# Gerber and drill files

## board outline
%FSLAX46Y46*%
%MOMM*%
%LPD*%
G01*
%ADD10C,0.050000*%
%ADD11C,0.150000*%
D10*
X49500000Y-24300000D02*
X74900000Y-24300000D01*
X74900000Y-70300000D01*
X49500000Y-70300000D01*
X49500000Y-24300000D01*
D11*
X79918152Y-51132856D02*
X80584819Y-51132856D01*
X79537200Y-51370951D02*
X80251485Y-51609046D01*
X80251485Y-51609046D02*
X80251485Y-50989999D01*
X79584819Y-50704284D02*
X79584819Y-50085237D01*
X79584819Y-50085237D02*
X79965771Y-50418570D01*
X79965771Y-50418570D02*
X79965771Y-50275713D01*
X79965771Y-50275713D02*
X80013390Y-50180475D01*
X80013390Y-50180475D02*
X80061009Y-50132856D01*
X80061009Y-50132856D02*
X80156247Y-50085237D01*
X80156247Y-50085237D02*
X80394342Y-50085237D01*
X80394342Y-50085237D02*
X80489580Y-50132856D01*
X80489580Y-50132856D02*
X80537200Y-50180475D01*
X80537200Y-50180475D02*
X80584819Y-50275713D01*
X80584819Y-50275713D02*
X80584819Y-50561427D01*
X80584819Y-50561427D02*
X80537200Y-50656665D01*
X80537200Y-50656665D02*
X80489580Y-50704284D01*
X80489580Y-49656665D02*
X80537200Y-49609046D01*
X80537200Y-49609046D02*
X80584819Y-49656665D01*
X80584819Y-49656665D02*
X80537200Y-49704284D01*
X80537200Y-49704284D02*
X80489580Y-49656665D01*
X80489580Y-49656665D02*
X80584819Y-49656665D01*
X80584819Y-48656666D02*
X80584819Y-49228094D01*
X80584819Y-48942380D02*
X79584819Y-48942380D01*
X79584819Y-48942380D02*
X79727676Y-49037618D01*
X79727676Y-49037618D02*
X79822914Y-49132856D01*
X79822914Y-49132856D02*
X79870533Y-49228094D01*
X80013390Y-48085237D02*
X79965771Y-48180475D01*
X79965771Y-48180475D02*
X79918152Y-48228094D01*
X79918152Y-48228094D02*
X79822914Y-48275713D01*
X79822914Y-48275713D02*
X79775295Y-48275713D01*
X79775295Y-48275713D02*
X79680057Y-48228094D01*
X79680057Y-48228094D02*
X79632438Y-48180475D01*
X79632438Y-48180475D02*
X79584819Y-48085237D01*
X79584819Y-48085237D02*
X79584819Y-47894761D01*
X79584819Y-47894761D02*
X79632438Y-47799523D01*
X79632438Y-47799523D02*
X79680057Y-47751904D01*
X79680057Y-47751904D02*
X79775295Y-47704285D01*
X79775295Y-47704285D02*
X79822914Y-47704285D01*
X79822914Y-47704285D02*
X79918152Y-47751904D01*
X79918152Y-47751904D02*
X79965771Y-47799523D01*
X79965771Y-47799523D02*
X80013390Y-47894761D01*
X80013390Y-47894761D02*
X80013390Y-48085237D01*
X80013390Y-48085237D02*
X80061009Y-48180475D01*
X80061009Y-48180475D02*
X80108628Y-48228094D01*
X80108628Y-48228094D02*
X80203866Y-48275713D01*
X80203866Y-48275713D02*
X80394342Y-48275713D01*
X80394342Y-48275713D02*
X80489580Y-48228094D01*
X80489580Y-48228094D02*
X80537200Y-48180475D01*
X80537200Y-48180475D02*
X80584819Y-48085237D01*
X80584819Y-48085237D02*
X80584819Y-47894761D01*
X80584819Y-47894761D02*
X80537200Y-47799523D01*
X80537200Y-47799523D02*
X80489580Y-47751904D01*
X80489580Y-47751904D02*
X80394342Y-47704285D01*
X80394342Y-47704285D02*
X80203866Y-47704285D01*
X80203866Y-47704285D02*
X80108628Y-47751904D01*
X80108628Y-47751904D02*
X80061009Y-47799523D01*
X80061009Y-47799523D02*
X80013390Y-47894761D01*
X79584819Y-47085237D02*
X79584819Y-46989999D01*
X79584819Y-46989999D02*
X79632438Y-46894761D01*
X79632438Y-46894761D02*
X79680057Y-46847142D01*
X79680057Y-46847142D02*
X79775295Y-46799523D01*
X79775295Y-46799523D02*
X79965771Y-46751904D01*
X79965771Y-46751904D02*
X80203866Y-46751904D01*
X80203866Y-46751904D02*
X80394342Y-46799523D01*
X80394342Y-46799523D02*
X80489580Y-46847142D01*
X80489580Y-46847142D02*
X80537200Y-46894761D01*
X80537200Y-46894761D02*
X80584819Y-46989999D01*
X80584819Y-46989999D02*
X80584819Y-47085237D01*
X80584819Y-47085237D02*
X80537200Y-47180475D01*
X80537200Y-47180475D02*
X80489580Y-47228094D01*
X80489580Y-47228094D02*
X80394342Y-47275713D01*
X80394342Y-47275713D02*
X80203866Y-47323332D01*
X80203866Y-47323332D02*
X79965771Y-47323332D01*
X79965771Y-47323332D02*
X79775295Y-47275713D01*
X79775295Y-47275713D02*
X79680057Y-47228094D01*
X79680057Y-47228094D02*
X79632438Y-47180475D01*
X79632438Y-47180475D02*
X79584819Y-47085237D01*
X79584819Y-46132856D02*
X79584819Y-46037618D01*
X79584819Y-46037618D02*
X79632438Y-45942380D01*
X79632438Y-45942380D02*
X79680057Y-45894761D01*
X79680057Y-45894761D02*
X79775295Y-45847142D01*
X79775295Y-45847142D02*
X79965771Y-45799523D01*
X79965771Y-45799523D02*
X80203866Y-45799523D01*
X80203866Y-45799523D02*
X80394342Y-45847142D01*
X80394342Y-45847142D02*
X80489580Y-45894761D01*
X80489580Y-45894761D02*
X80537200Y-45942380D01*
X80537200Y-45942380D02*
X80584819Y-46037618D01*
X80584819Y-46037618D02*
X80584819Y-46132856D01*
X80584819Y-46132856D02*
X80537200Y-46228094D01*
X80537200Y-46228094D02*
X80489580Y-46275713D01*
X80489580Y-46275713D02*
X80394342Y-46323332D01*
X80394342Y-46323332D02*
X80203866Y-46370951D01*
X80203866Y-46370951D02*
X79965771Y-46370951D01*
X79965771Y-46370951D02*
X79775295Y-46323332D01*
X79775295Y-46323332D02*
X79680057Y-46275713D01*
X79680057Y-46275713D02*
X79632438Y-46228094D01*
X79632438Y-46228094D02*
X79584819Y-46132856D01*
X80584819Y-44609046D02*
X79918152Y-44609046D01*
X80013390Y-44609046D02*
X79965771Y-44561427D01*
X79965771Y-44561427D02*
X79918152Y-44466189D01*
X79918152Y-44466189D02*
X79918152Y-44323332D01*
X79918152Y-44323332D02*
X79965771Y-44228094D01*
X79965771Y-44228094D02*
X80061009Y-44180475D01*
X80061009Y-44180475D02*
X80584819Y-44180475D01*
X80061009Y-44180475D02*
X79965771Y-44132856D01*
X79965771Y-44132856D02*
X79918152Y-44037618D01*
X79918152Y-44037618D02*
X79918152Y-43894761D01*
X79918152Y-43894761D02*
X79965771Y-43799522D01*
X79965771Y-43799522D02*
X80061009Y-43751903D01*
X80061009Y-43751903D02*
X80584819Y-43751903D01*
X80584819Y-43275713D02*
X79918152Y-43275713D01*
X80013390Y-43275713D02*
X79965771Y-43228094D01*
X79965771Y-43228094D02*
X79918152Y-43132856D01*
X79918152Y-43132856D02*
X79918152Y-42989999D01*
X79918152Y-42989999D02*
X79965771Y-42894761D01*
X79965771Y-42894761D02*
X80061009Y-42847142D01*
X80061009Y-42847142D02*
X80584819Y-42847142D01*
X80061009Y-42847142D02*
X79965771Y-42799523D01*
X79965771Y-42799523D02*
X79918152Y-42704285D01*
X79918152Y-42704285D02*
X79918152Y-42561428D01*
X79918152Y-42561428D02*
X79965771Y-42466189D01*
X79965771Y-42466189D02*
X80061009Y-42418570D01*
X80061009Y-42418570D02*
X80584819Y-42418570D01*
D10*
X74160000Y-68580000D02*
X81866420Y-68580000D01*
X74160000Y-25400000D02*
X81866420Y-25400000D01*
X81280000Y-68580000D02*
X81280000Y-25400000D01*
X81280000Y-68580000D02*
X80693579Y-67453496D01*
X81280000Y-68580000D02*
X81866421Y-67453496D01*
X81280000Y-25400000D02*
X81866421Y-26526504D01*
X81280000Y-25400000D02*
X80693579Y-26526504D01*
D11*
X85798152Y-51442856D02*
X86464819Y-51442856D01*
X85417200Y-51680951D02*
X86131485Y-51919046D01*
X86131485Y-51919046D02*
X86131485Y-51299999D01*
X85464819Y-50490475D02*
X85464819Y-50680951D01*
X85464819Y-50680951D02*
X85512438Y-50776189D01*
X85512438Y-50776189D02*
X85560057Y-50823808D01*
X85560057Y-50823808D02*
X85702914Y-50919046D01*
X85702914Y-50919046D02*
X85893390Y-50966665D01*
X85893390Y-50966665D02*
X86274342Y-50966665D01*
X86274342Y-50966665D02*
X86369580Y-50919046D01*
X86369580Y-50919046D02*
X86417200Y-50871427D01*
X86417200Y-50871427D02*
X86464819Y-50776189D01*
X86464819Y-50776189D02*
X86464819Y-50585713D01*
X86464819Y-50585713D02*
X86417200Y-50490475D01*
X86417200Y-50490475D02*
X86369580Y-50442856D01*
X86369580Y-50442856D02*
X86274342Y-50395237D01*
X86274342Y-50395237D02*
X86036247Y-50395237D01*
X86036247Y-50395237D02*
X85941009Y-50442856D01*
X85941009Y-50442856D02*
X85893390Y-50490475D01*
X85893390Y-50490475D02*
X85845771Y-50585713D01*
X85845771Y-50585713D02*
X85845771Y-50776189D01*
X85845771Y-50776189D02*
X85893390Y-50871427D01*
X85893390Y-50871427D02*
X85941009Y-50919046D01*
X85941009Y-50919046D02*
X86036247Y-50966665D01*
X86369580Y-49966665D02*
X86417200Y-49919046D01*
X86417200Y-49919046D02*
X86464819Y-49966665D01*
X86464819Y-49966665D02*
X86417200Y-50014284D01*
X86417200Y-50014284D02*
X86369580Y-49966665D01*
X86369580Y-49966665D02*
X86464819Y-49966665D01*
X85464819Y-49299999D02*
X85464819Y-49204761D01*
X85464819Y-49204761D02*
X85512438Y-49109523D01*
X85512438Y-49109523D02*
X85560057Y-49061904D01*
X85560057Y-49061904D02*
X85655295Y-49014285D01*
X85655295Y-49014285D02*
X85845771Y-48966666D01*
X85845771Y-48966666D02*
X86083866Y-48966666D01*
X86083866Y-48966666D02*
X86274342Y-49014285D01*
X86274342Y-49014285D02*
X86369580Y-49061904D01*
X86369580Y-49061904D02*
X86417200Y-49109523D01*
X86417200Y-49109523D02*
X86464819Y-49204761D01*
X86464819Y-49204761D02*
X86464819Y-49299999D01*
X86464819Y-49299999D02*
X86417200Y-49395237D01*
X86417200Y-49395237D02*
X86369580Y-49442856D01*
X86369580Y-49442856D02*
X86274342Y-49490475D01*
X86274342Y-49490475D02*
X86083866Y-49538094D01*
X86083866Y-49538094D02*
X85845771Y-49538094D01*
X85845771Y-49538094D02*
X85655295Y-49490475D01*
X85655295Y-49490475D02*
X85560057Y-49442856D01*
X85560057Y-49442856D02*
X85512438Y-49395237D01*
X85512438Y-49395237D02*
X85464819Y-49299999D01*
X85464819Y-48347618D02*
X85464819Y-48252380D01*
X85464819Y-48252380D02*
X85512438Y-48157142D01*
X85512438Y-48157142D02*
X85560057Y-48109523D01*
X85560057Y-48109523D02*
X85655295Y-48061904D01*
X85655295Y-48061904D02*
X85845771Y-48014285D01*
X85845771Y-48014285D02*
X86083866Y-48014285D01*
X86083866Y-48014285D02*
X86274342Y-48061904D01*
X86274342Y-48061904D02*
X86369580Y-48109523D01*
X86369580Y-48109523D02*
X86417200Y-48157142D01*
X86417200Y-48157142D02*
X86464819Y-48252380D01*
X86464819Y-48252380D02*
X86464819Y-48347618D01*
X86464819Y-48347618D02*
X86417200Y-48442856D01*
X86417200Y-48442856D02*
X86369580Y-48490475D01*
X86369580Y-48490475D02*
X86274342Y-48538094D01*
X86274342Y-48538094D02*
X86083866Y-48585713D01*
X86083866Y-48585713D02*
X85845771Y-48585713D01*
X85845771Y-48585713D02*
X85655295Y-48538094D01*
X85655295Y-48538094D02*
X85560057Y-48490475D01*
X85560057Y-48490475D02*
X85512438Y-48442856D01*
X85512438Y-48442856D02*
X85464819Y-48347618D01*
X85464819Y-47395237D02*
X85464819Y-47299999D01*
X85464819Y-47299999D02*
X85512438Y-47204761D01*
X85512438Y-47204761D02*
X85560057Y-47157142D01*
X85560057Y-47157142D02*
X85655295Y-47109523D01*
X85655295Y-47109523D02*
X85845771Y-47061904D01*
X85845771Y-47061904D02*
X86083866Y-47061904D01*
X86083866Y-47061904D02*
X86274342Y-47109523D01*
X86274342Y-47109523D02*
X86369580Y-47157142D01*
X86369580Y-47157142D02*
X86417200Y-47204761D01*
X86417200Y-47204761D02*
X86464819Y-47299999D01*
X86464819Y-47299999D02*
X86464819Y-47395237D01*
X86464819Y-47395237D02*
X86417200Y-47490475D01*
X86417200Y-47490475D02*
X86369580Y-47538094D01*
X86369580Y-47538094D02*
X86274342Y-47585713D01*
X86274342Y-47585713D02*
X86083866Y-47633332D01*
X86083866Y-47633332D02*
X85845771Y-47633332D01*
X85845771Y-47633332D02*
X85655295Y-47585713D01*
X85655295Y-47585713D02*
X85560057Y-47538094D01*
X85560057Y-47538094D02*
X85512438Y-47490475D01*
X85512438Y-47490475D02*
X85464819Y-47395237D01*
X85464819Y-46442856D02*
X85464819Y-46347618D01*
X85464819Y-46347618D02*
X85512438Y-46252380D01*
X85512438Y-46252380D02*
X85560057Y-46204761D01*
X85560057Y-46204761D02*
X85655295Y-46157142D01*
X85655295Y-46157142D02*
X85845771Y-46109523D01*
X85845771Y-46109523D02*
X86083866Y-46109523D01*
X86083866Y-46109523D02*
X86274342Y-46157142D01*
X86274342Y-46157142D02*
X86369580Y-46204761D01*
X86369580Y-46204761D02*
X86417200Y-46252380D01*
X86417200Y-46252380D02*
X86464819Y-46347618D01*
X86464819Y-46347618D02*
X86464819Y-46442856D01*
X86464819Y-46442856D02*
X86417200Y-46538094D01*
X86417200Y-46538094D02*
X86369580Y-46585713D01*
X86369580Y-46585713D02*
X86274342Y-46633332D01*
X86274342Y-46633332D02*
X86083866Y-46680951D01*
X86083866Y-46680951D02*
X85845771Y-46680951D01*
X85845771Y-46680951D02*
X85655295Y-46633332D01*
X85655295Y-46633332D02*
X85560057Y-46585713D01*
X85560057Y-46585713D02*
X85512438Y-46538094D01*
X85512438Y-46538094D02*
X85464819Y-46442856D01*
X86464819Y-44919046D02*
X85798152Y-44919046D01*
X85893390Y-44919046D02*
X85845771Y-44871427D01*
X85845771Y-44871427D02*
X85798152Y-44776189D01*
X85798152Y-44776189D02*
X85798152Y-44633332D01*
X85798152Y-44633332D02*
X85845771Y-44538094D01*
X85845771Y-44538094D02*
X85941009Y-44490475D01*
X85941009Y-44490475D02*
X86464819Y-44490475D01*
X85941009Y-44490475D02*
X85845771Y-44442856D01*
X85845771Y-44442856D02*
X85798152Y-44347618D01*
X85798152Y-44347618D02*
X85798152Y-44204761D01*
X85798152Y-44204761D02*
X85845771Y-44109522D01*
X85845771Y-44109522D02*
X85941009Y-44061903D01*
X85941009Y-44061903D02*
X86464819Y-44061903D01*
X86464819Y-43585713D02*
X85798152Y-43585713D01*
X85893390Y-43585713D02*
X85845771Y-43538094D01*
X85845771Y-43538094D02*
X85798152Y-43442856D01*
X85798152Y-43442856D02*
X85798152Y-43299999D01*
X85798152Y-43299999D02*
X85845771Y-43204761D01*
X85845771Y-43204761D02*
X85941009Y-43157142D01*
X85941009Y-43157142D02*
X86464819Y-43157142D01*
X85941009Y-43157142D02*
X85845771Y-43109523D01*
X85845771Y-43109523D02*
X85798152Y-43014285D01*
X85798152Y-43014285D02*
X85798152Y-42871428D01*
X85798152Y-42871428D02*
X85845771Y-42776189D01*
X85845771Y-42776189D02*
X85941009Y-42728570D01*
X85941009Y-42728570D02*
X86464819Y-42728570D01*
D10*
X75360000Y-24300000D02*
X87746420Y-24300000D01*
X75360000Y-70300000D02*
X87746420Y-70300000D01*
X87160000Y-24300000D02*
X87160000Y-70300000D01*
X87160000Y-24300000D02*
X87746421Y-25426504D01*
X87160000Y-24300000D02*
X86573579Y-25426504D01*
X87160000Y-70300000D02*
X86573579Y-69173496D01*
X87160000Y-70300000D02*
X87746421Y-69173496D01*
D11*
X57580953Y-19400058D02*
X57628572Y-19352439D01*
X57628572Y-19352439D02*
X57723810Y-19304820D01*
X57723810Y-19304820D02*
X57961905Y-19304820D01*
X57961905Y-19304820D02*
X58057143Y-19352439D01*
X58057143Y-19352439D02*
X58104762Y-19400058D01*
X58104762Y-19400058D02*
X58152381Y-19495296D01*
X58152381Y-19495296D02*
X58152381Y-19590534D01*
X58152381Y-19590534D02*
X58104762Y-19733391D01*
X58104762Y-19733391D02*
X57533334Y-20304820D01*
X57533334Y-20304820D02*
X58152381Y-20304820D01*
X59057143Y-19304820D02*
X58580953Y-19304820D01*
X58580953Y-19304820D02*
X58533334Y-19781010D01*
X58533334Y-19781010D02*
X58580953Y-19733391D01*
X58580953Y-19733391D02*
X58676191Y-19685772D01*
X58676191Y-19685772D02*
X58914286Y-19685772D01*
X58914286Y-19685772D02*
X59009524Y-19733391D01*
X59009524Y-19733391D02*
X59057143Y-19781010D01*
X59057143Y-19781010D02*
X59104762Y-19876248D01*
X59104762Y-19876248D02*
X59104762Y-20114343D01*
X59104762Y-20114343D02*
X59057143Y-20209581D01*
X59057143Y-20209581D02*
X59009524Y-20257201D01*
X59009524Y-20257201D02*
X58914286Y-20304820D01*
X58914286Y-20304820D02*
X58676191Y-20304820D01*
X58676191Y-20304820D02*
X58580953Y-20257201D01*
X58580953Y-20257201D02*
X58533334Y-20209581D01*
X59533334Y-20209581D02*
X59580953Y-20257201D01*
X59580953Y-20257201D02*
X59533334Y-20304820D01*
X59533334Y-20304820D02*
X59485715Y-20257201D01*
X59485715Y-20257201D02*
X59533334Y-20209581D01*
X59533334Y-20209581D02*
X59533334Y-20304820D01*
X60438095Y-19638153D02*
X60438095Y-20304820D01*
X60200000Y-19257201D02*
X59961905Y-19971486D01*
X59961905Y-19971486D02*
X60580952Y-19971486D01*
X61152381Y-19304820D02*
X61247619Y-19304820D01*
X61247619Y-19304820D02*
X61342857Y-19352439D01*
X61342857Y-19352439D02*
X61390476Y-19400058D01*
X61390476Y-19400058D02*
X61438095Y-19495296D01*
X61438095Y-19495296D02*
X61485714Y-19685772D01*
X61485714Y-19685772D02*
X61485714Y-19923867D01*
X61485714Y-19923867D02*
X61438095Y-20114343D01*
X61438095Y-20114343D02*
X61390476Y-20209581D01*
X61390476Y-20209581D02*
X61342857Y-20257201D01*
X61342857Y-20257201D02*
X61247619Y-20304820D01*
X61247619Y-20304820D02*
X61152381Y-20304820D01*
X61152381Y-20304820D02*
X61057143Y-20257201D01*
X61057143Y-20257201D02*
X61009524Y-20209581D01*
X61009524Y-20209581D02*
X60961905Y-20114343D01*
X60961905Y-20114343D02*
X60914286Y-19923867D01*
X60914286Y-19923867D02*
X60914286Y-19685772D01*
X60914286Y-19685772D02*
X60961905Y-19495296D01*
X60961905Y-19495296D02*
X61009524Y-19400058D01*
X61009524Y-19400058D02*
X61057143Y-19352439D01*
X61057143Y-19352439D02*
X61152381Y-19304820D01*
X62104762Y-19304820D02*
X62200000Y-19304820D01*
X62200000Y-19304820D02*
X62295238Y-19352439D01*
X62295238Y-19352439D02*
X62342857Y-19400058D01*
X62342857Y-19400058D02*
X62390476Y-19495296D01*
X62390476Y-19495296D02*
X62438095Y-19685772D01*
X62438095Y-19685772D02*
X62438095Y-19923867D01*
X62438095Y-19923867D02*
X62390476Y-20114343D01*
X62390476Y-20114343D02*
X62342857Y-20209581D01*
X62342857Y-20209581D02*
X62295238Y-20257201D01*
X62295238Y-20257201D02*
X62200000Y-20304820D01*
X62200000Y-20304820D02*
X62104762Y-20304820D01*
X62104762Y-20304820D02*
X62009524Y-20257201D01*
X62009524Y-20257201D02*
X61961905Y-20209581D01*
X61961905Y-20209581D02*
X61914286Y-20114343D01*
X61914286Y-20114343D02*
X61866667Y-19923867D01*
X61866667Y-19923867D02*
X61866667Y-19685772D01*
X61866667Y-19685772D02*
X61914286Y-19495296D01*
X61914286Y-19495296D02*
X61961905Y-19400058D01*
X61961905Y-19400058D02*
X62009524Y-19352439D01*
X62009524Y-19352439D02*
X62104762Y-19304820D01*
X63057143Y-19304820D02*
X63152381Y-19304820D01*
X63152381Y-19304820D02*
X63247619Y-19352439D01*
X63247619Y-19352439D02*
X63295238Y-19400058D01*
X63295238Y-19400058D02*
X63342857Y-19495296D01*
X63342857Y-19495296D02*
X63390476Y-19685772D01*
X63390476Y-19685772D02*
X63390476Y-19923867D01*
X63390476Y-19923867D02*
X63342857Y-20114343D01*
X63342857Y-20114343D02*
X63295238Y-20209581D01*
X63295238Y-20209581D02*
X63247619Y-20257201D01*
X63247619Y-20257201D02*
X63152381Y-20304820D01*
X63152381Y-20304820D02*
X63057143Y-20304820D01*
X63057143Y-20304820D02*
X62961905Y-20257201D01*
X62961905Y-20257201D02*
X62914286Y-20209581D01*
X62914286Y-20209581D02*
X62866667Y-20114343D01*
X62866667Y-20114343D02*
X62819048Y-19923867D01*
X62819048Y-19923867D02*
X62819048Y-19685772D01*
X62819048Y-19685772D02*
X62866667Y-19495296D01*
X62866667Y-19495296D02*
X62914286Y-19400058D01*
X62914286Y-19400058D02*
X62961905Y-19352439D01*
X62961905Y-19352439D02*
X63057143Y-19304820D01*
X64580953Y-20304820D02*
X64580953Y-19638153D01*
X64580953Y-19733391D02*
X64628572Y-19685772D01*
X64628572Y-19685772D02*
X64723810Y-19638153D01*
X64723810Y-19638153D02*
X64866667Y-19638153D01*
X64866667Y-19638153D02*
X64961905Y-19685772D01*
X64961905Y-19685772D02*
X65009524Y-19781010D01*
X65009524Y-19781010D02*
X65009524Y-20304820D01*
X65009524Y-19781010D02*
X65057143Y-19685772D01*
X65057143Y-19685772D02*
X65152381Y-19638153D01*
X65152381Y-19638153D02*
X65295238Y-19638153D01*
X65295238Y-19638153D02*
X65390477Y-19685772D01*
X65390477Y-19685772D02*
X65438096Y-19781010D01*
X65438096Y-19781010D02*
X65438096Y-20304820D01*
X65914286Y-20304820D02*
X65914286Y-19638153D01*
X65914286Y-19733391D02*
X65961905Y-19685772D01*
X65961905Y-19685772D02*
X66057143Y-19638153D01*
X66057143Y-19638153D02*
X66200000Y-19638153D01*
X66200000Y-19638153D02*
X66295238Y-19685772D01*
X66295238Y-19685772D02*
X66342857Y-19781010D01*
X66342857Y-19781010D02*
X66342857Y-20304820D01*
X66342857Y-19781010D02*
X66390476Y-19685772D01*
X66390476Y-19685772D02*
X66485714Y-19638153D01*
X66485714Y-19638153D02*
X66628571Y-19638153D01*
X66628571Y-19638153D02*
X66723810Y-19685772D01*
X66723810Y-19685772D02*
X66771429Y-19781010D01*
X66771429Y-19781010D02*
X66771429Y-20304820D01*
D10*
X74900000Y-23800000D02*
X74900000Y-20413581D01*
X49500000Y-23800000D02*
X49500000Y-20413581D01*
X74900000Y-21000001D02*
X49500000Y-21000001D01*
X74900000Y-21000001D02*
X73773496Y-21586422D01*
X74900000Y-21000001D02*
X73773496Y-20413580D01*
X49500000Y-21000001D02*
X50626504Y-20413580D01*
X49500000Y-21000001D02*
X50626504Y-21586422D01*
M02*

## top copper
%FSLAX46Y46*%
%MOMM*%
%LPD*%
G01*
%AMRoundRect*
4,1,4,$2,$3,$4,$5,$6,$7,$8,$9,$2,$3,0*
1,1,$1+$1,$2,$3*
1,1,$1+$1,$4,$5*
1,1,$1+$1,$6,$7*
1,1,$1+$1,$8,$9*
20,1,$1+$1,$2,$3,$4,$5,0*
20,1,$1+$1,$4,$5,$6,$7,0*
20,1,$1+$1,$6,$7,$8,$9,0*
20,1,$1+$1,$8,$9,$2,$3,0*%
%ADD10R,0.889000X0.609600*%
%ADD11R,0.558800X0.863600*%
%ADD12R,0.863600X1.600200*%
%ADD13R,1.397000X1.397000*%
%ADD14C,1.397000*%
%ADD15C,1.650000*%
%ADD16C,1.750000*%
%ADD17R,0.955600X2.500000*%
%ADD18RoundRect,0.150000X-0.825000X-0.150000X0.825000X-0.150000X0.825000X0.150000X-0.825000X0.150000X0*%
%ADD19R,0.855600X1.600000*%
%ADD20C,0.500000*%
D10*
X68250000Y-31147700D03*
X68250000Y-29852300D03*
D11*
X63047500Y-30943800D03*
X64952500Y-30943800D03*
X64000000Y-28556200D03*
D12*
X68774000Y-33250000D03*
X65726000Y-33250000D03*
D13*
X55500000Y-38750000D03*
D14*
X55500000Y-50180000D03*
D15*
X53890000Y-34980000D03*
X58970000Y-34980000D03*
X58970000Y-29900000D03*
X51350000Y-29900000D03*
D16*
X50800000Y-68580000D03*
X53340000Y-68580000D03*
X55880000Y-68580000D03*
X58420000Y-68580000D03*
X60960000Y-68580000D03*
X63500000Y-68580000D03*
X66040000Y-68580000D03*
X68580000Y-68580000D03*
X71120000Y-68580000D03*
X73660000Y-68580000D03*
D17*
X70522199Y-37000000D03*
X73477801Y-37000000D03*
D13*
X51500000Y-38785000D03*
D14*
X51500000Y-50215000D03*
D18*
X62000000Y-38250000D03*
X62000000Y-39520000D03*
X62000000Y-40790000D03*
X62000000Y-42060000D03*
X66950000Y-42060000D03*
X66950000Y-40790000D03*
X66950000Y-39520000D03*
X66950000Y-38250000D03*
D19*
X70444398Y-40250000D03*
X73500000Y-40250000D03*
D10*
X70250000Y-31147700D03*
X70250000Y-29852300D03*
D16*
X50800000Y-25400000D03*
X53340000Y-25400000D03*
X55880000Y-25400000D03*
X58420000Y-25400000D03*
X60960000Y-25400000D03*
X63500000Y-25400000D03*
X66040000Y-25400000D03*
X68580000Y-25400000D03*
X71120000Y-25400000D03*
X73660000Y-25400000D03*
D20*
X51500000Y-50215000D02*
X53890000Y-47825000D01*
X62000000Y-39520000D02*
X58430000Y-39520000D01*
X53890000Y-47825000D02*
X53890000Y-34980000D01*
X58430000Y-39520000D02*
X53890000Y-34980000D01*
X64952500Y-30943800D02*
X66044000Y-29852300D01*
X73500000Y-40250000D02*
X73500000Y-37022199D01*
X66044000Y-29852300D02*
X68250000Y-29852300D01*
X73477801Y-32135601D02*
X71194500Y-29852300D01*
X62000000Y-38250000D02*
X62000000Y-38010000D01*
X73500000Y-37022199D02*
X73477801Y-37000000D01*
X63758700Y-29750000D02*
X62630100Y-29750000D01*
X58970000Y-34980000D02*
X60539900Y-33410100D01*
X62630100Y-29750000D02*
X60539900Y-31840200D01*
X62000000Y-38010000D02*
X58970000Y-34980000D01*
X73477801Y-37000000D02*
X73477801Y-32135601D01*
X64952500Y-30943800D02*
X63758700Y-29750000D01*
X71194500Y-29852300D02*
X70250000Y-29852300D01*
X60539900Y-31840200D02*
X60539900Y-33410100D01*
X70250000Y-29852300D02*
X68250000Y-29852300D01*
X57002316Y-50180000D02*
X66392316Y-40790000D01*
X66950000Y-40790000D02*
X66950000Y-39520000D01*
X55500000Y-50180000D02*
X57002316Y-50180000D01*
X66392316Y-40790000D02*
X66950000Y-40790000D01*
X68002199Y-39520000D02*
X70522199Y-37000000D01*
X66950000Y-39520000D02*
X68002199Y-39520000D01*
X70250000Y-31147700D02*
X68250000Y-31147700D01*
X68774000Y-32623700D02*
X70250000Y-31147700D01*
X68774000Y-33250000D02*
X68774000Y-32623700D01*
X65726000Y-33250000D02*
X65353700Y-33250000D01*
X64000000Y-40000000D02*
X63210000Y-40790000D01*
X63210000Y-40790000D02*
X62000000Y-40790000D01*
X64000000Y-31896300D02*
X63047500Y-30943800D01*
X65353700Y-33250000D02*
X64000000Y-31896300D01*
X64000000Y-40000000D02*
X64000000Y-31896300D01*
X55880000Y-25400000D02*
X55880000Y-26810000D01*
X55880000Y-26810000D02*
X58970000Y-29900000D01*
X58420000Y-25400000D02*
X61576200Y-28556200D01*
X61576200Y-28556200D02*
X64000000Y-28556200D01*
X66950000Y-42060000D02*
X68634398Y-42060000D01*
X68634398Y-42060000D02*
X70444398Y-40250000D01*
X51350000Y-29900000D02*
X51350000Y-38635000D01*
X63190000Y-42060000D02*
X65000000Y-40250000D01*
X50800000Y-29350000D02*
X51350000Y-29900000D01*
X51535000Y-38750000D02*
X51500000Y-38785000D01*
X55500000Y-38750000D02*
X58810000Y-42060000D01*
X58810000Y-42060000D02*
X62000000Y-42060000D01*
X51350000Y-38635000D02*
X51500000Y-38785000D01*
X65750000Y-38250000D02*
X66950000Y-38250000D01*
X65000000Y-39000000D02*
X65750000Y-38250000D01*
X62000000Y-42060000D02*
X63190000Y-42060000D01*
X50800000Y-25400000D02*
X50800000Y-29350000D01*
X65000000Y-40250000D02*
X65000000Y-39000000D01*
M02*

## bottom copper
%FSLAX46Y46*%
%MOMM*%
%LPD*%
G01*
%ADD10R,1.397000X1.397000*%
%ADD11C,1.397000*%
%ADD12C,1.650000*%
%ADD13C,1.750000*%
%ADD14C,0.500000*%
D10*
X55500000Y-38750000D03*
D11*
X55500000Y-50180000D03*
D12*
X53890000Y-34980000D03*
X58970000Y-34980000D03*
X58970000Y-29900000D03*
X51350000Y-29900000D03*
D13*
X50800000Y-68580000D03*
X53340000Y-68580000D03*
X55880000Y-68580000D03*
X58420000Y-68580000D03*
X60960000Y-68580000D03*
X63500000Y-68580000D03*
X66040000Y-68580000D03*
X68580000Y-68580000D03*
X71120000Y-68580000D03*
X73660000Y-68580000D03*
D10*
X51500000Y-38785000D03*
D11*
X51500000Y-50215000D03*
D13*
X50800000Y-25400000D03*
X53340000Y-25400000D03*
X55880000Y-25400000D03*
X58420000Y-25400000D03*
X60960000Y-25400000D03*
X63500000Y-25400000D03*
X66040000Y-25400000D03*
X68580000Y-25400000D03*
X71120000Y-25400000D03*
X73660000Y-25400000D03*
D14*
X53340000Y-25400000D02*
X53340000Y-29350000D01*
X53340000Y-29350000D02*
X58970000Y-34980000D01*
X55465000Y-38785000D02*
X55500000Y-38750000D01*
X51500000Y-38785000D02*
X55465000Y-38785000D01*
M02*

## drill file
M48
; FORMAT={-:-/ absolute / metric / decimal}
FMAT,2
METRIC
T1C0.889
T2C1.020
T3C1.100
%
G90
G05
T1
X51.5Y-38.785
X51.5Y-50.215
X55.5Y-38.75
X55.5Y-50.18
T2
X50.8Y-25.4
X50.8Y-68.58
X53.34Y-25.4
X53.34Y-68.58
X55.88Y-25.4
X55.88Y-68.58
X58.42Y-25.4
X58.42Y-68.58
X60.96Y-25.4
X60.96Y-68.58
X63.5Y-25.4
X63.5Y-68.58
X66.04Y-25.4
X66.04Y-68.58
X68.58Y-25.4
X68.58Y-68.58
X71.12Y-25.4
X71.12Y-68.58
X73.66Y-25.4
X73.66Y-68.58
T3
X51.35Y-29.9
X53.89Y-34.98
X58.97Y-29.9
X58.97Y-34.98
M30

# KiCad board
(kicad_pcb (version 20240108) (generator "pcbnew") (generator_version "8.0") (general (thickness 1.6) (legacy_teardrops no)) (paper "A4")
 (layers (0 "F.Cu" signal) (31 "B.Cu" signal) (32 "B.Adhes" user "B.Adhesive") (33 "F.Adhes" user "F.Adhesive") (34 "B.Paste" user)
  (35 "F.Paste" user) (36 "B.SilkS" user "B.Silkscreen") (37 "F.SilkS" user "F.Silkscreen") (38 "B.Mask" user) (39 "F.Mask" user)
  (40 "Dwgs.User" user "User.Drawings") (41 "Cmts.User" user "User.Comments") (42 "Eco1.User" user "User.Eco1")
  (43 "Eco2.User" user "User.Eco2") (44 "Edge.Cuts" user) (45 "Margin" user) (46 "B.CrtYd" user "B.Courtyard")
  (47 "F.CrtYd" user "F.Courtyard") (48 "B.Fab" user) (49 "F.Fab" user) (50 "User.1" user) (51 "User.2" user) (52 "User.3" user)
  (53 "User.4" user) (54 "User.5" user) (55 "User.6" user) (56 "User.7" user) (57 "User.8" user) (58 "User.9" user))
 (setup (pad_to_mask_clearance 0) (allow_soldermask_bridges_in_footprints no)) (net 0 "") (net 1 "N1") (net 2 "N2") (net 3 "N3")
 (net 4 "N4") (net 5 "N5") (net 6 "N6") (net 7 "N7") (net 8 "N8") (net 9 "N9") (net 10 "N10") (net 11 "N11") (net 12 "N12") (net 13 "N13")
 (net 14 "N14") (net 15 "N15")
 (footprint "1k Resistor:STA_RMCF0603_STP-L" (layer "F.Cu") (at 68.25 30.5 90)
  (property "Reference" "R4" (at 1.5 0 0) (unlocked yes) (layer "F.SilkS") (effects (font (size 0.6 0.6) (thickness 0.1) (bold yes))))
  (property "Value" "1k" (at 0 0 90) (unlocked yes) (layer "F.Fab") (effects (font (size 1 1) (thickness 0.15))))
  (pad "1" smd rect (at -0.6477 0 90) (size 0.6096 0.889) (layers "F.Cu" "F.Paste" "F.Mask") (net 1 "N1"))
  (pad "2" smd rect (at 0.6477 0 90) (size 0.6096 0.889) (layers "F.Cu" "F.Paste" "F.Mask") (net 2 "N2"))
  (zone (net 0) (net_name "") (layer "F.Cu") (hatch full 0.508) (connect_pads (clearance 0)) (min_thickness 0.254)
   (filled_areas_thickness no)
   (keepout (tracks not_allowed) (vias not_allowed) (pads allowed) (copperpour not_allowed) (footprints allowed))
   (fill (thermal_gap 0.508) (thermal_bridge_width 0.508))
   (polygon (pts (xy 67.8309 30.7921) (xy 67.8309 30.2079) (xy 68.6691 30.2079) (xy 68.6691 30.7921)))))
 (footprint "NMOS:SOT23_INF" (layer "F.Cu") (at 64 29.75)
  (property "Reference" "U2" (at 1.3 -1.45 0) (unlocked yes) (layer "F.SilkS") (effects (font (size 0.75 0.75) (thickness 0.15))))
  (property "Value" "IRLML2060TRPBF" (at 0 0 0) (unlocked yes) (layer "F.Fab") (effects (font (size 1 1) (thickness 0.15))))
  (pad "1" smd rect (at -0.9525 1.1938) (size 0.5588 0.8636) (layers "F.Cu" "F.Paste" "F.Mask") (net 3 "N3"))
  (pad "2" smd rect (at 0.9525 1.1938) (size 0.5588 0.8636) (layers "F.Cu" "F.Paste" "F.Mask") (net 2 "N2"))
  (pad "3" smd rect (at 0 -1.1938) (size 0.5588 0.8636) (layers "F.Cu" "F.Paste" "F.Mask") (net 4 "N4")))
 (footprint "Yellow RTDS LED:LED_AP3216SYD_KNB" (layer "F.Cu") (at 67.25 33.25 180)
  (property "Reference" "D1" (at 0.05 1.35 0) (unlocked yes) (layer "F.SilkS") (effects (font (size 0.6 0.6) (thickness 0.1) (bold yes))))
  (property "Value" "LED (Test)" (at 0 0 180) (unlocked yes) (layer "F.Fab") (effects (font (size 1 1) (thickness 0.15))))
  (pad "1" smd rect (at -1.524 0 180) (size 0.8636 1.6002) (layers "F.Cu" "F.Paste" "F.Mask") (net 1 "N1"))
  (pad "2" smd rect (at 1.524 0 180) (size 0.8636 1.6002) (layers "F.Cu" "F.Paste" "F.Mask") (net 3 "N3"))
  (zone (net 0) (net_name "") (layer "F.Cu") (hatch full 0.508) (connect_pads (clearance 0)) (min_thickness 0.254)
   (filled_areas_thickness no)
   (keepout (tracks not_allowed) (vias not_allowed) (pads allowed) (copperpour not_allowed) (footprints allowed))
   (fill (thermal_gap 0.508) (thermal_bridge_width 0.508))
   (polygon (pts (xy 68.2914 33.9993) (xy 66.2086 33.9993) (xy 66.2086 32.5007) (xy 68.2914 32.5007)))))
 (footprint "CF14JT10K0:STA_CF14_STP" (layer "F.Cu") (at 55.5 38.75 -90)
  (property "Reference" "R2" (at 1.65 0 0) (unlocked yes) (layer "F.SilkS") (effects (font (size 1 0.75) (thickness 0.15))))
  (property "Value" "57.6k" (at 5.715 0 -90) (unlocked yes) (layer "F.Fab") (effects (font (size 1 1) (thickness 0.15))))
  (pad "1" thru_hole rect (at 0 0 270) (size 1.397 1.397) (drill 0.889) (layers "*.Cu" "*.Mask") (remove_unused_layers no) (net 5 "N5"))
  (pad "2" thru_hole circle (at 11.43 0 270) (size 1.397 1.397) (drill 0.889) (layers "*.Cu" "*.Mask") (remove_unused_layers no)
   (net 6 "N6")))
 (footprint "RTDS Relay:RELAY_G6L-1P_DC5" (layer "F.Cu") (at 55.16 32.44)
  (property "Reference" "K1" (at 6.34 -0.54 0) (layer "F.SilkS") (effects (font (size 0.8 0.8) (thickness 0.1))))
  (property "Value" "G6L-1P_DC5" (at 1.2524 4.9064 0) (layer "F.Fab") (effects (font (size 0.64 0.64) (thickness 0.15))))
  (pad "2" thru_hole circle (at -1.27 2.54) (size 1.65 1.65) (drill 1.1) (layers "*.Cu" "*.Mask") (remove_unused_layers no) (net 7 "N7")
   (solder_mask_margin 0.102))
  (pad "4" thru_hole circle (at 3.81 2.54) (size 1.65 1.65) (drill 1.1) (layers "*.Cu" "*.Mask") (remove_unused_layers no) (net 2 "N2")
   (solder_mask_margin 0.102))
  (pad "5" thru_hole circle (at 3.81 -2.54) (size 1.65 1.65) (drill 1.1) (layers "*.Cu" "*.Mask") (remove_unused_layers no) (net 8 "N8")
   (solder_mask_margin 0.102))
  (pad "8" thru_hole circle (at -3.81 -2.54) (size 1.65 1.65) (drill 1.1) (layers "*.Cu" "*.Mask") (remove_unused_layers no) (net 5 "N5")
   (solder_mask_margin 0.102)))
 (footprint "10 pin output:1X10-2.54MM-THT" (layer "F.Cu") (at 50.8 68.58)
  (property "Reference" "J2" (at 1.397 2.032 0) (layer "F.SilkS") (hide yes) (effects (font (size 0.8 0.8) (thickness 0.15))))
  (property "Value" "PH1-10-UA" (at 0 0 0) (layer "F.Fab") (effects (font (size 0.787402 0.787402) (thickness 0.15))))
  (pad "1" thru_hole circle (at 0 0) (size 1.75 1.75) (drill 1.02) (layers "*.Cu" "*.Mask") (remove_unused_layers no)
   (solder_mask_margin 0.102))
  (pad "2" thru_hole circle (at 2.54 0) (size 1.75 1.75) (drill 1.02) (layers "*.Cu" "*.Mask") (remove_unused_layers no)
   (solder_mask_margin 0.102))
  (pad "3" thru_hole circle (at 5.08 0) (size 1.75 1.75) (drill 1.02) (layers "*.Cu" "*.Mask") (remove_unused_layers no)
   (solder_mask_margin 0.102))
  (pad "4" thru_hole circle (at 7.62 0) (size 1.75 1.75) (drill 1.02) (layers "*.Cu" "*.Mask") (remove_unused_layers no)
   (solder_mask_margin 0.102))
  (pad "5" thru_hole circle (at 10.16 0) (size 1.75 1.75) (drill 1.02) (layers "*.Cu" "*.Mask") (remove_unused_layers no)
   (solder_mask_margin 0.102))
  (pad "6" thru_hole circle (at 12.7 0) (size 1.75 1.75) (drill 1.02) (layers "*.Cu" "*.Mask") (remove_unused_layers no)
   (solder_mask_margin 0.102))
  (pad "7" thru_hole circle (at 15.24 0) (size 1.75 1.75) (drill 1.02) (layers "*.Cu" "*.Mask") (remove_unused_layers no)
   (solder_mask_margin 0.102))
  (pad "8" thru_hole circle (at 17.78 0) (size 1.75 1.75) (drill 1.02) (layers "*.Cu" "*.Mask") (remove_unused_layers no)
   (solder_mask_margin 0.102))
  (pad "9" thru_hole circle (at 20.32 0) (size 1.75 1.75) (drill 1.02) (layers "*.Cu" "*.Mask") (remove_unused_layers no)
   (solder_mask_margin 0.102))
  (pad "10" thru_hole circle (at 22.86 0) (size 1.75 1.75) (drill 1.02) (layers "*.Cu" "*.Mask") (remove_unused_layers no)
   (solder_mask_margin 0.102)))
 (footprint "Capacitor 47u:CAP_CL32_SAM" (layer "F.Cu") (at 72 37)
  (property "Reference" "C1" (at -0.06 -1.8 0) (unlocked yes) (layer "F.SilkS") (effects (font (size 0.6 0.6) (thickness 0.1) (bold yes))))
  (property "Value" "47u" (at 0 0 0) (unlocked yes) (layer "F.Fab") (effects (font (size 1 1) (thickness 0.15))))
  (pad "1" smd rect (at -1.477801 0) (size 0.9556 2.5) (layers "F.Cu" "F.Paste" "F.Mask") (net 6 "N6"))
  (pad "2" smd rect (at 1.477801 0) (size 0.9556 2.5) (layers "F.Cu" "F.Paste" "F.Mask") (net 2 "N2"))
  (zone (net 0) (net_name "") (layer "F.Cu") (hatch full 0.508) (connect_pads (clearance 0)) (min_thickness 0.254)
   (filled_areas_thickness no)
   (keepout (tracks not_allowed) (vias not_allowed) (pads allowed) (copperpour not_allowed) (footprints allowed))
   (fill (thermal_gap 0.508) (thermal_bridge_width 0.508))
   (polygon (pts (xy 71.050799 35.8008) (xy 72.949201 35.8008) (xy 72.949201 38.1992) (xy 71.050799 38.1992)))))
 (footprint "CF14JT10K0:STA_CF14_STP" (layer "F.Cu") (at 51.5 38.785 -90)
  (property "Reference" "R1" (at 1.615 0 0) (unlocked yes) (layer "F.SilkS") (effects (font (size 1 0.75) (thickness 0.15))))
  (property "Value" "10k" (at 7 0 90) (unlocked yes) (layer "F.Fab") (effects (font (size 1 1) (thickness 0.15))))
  (pad "1" thru_hole rect (at 0 0 270) (size 1.397 1.397) (drill 0.889) (layers "*.Cu" "*.Mask") (remove_unused_layers no) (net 5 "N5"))
  (pad "2" thru_hole circle (at 11.43 0 270) (size 1.397 1.397) (drill 0.889) (layers "*.Cu" "*.Mask") (remove_unused_layers no)
   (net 7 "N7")))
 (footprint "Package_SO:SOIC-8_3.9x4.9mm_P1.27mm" (layer "F.Cu") (at 64.475 40.155)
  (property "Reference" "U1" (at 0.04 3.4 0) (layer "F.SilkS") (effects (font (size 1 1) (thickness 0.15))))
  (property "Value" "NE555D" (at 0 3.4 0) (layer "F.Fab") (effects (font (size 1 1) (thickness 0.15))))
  (pad "1" smd roundrect (at -2.475 -1.905) (size 1.95 0.6) (layers "F.Cu" "F.Paste" "F.Mask") (roundrect_rratio 0.25) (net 2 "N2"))
  (pad "2" smd roundrect (at -2.475 -0.635) (size 1.95 0.6) (layers "F.Cu" "F.Paste" "F.Mask") (roundrect_rratio 0.25) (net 7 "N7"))
  (pad "3" smd roundrect (at -2.475 0.635) (size 1.95 0.6) (layers "F.Cu" "F.Paste" "F.Mask") (roundrect_rratio 0.25) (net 3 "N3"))
  (pad "4" smd roundrect (at -2.475 1.905) (size 1.95 0.6) (layers "F.Cu" "F.Paste" "F.Mask") (roundrect_rratio 0.25) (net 5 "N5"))
  (pad "5" smd roundrect (at 2.475 1.905) (size 1.95 0.6) (layers "F.Cu" "F.Paste" "F.Mask") (roundrect_rratio 0.25) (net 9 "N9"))
  (pad "6" smd roundrect (at 2.475 0.635) (size 1.95 0.6) (layers "F.Cu" "F.Paste" "F.Mask") (roundrect_rratio 0.25) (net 6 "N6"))
  (pad "7" smd roundrect (at 2.475 -0.635) (size 1.95 0.6) (layers "F.Cu" "F.Paste" "F.Mask") (roundrect_rratio 0.25) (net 6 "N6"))
  (pad "8" smd roundrect (at 2.475 -1.905) (size 1.95 0.6) (layers "F.Cu" "F.Paste" "F.Mask") (roundrect_rratio 0.25) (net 5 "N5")))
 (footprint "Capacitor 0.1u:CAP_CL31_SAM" (layer "F.Cu") (at 71.972199 40.25)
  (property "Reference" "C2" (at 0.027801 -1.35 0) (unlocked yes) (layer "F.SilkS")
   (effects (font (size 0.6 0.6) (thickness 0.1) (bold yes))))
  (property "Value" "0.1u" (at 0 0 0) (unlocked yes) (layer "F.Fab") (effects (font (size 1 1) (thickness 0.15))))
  (pad "1" smd rect (at -1.527801 0) (size 0.8556 1.6) (layers "F.Cu" "F.Paste" "F.Mask") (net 9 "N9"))
  (pad "2" smd rect (at 1.527801 0) (size 0.8556 1.6) (layers "F.Cu" "F.Paste" "F.Mask") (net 2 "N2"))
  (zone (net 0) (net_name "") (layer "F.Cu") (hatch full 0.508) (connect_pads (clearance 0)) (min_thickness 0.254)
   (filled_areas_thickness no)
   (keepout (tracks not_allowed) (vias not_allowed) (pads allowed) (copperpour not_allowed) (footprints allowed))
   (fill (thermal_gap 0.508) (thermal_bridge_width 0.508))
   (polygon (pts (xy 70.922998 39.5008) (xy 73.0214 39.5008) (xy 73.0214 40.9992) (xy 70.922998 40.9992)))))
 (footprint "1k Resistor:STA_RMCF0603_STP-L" (layer "F.Cu") (at 70.25 30.5 90)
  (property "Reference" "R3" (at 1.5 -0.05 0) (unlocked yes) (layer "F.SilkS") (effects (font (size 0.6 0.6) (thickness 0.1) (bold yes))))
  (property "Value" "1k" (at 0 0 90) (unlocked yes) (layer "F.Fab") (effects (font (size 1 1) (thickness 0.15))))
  (pad "1" smd rect (at -0.6477 0 90) (size 0.6096 0.889) (layers "F.Cu" "F.Paste" "F.Mask") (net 1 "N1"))
  (pad "2" smd rect (at 0.6477 0 90) (size 0.6096 0.889) (layers "F.Cu" "F.Paste" "F.Mask") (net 2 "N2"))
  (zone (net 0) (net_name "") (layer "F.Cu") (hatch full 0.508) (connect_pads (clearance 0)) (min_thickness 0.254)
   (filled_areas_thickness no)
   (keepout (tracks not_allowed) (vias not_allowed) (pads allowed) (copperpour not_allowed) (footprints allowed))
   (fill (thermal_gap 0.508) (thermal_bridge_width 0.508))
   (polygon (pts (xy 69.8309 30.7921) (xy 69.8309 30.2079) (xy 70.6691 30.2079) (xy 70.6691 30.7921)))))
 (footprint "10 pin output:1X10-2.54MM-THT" (layer "F.Cu") (at 50.8 25.4)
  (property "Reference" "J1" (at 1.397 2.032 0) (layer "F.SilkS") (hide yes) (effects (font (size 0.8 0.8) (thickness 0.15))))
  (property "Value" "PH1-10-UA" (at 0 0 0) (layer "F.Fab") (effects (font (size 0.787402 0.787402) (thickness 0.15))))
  (pad "1" thru_hole circle (at 0 0) (size 1.75 1.75) (drill 1.02) (layers "*.Cu" "*.Mask") (remove_unused_layers no) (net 5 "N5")
   (solder_mask_margin 0.102))
  (pad "2" thru_hole circle (at 2.54 0) (size 1.75 1.75) (drill 1.02) (layers "*.Cu" "*.Mask") (remove_unused_layers no) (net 2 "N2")
   (solder_mask_margin 0.102))
  (pad "3" thru_hole circle (at 5.08 0) (size 1.75 1.75) (drill 1.02) (layers "*.Cu" "*.Mask") (remove_unused_layers no) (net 8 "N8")
   (solder_mask_margin 0.102))
  (pad "4" thru_hole circle (at 7.62 0) (size 1.75 1.75) (drill 1.02) (layers "*.Cu" "*.Mask") (remove_unused_layers no) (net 4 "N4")
   (solder_mask_margin 0.102))
  (pad "5" thru_hole circle (at 10.16 0) (size 1.75 1.75) (drill 1.02) (layers "*.Cu" "*.Mask") (remove_unused_layers no) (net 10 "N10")
   (solder_mask_margin 0.102))
  (pad "6" thru_hole circle (at 12.7 0) (size 1.75 1.75) (drill 1.02) (layers "*.Cu" "*.Mask") (remove_unused_layers no) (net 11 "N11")
   (solder_mask_margin 0.102))
  (pad "7" thru_hole circle (at 15.24 0) (size 1.75 1.75) (drill 1.02) (layers "*.Cu" "*.Mask") (remove_unused_layers no) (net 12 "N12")
   (solder_mask_margin 0.102))
  (pad "8" thru_hole circle (at 17.78 0) (size 1.75 1.75) (drill 1.02) (layers "*.Cu" "*.Mask") (remove_unused_layers no) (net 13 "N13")
   (solder_mask_margin 0.102))
  (pad "9" thru_hole circle (at 20.32 0) (size 1.75 1.75) (drill 1.02) (layers "*.Cu" "*.Mask") (remove_unused_layers no) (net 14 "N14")
   (solder_mask_margin 0.102))
  (pad "10" thru_hole circle (at 22.86 0) (size 1.75 1.75) (drill 1.02) (layers "*.Cu" "*.Mask") (remove_unused_layers no) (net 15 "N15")
   (solder_mask_margin 0.102)))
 (gr_rect (start 49.5 24.3) (end 74.9 70.3) (stroke (width 0.05) (type default)) (fill none) (layer "Edge.Cuts"))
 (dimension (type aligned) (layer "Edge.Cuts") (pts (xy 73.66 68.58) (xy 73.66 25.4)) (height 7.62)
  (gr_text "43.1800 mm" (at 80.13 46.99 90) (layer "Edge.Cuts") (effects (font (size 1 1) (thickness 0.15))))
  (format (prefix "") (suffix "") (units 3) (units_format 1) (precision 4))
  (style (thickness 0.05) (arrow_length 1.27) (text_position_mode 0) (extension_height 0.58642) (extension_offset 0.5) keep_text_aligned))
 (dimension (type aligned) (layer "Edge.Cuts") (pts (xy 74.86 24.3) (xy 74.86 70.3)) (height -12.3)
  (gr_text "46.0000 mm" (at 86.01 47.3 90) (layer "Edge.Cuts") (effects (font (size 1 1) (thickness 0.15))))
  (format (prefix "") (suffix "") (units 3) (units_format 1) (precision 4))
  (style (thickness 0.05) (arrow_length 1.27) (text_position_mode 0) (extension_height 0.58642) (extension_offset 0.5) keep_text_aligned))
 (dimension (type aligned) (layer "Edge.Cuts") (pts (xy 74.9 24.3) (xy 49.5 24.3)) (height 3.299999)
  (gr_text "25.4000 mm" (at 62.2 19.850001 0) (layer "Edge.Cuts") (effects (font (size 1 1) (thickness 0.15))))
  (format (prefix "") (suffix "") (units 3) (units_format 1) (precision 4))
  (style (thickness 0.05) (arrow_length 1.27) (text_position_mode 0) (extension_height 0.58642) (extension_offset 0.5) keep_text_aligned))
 (segment (start 51.5 50.215) (end 53.89 47.825) (width 0.5) (layer "F.Cu") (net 7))
 (segment (start 62 39.52) (end 58.43 39.52) (width 0.5) (layer "F.Cu") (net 7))
 (segment (start 53.89 47.825) (end 53.89 34.98) (width 0.5) (layer "F.Cu") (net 7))
 (segment (start 58.43 39.52) (end 53.89 34.98) (width 0.5) (layer "F.Cu") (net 7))
 (segment (start 64.9525 30.9438) (end 66.044 29.8523) (width 0.5) (layer "F.Cu") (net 2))
 (segment (start 73.5 40.25) (end 73.5 37.022199) (width 0.5) (layer "F.Cu") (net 2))
 (segment (start 66.044 29.8523) (end 68.25 29.8523) (width 0.5) (layer "F.Cu") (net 2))
 (segment (start 73.477801 32.135601) (end 71.1945 29.8523) (width 0.5) (layer "F.Cu") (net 2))
 (segment (start 62 38.25) (end 62 38.01) (width 0.5) (layer "F.Cu") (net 2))
 (segment (start 73.5 37.022199) (end 73.477801 37) (width 0.5) (layer "F.Cu") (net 2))
 (segment (start 63.7587 29.75) (end 62.6301 29.75) (width 0.5) (layer "F.Cu") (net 2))
 (segment (start 58.97 34.98) (end 60.5399 33.4101) (width 0.5) (layer "F.Cu") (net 2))
 (segment (start 62.6301 29.75) (end 60.5399 31.8402) (width 0.5) (layer "F.Cu") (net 2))
 (segment (start 62 38.01) (end 58.97 34.98) (width 0.5) (layer "F.Cu") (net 2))
 (segment (start 73.477801 37) (end 73.477801 32.135601) (width 0.5) (layer "F.Cu") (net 2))
 (segment (start 64.9525 30.9438) (end 63.7587 29.75) (width 0.5) (layer "F.Cu") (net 2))
 (segment (start 71.1945 29.8523) (end 70.25 29.8523) (width 0.5) (layer "F.Cu") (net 2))
 (segment (start 60.5399 31.8402) (end 60.5399 33.4101) (width 0.5) (layer "F.Cu") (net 2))
 (segment (start 70.25 29.8523) (end 68.25 29.8523) (width 0.5) (layer "F.Cu") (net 2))
 (segment (start 53.34 25.4) (end 53.34 29.35) (width 0.5) (layer "B.Cu") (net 2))
 (segment (start 53.34 29.35) (end 58.97 34.98) (width 0.5) (layer "B.Cu") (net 2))
 (segment (start 57.002316 50.18) (end 66.392316 40.79) (width 0.5) (layer "F.Cu") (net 6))
 (segment (start 66.95 40.79) (end 66.95 39.52) (width 0.5) (layer "F.Cu") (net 6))
 (segment (start 55.5 50.18) (end 57.002316 50.18) (width 0.5) (layer "F.Cu") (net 6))
 (segment (start 66.392316 40.79) (end 66.95 40.79) (width 0.5) (layer "F.Cu") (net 6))
 (segment (start 68.002199 39.52) (end 70.522199 37) (width 0.5) (layer "F.Cu") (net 6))
 (segment (start 66.95 39.52) (end 68.002199 39.52) (width 0.5) (layer "F.Cu") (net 6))
 (segment (start 70.25 31.1477) (end 68.25 31.1477) (width 0.5) (layer "F.Cu") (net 1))
 (segment (start 68.774 32.6237) (end 70.25 31.1477) (width 0.5) (layer "F.Cu") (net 1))
 (segment (start 68.774 33.25) (end 68.774 32.6237) (width 0.5) (layer "F.Cu") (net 1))
 (segment (start 65.726 33.25) (end 65.3537 33.25) (width 0.5) (layer "F.Cu") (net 3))
 (segment (start 64 40) (end 63.21 40.79) (width 0.5) (layer "F.Cu") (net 3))
 (segment (start 63.21 40.79) (end 62 40.79) (width 0.5) (layer "F.Cu") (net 3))
 (segment (start 64 31.8963) (end 63.0475 30.9438) (width 0.5) (layer "F.Cu") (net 3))
 (segment (start 65.3537 33.25) (end 64 31.8963) (width 0.5) (layer "F.Cu") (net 3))
 (segment (start 64 40) (end 64 31.8963) (width 0.5) (layer "F.Cu") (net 3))
 (segment (start 55.88 25.4) (end 55.88 26.81) (width 0.5) (layer "F.Cu") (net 8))
 (segment (start 55.88 26.81) (end 58.97 29.9) (width 0.5) (layer "F.Cu") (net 8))
 (segment (start 58.42 25.4) (end 61.5762 28.5562) (width 0.5) (layer "F.Cu") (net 4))
 (segment (start 61.5762 28.5562) (end 64 28.5562) (width 0.5) (layer "F.Cu") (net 4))
 (segment (start 66.95 42.06) (end 68.634398 42.06) (width 0.5) (layer "F.Cu") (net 9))
 (segment (start 68.634398 42.06) (end 70.444398 40.25) (width 0.5) (layer "F.Cu") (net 9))
 (segment (start 51.35 29.9) (end 51.35 38.635) (width 0.5) (layer "F.Cu") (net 5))
 (segment (start 63.19 42.06) (end 65 40.25) (width 0.5) (layer "F.Cu") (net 5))
 (segment (start 50.8 29.35) (end 51.35 29.9) (width 0.5) (layer "F.Cu") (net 5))
 (segment (start 51.535 38.75) (end 51.5 38.785) (width 0.5) (layer "F.Cu") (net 5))
 (segment (start 55.5 38.75) (end 58.81 42.06) (width 0.5) (layer "F.Cu") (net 5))
 (segment (start 58.81 42.06) (end 62 42.06) (width 0.5) (layer "F.Cu") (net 5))
 (segment (start 51.35 38.635) (end 51.5 38.785) (width 0.5) (layer "F.Cu") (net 5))
 (segment (start 65.75 38.25) (end 66.95 38.25) (width 0.5) (layer "F.Cu") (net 5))
 (segment (start 65 39) (end 65.75 38.25) (width 0.5) (layer "F.Cu") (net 5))
 (segment (start 62 42.06) (end 63.19 42.06) (width 0.5) (layer "F.Cu") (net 5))
 (segment (start 50.8 25.4) (end 50.8 29.35) (width 0.5) (layer "F.Cu") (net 5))
 (segment (start 65 40.25) (end 65 39) (width 0.5) (layer "F.Cu") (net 5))
 (segment (start 55.465 38.785) (end 55.5 38.75) (width 0.5) (layer "B.Cu") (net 5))
 (segment (start 51.5 38.785) (end 55.465 38.785) (width 0.5) (layer "B.Cu") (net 5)))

